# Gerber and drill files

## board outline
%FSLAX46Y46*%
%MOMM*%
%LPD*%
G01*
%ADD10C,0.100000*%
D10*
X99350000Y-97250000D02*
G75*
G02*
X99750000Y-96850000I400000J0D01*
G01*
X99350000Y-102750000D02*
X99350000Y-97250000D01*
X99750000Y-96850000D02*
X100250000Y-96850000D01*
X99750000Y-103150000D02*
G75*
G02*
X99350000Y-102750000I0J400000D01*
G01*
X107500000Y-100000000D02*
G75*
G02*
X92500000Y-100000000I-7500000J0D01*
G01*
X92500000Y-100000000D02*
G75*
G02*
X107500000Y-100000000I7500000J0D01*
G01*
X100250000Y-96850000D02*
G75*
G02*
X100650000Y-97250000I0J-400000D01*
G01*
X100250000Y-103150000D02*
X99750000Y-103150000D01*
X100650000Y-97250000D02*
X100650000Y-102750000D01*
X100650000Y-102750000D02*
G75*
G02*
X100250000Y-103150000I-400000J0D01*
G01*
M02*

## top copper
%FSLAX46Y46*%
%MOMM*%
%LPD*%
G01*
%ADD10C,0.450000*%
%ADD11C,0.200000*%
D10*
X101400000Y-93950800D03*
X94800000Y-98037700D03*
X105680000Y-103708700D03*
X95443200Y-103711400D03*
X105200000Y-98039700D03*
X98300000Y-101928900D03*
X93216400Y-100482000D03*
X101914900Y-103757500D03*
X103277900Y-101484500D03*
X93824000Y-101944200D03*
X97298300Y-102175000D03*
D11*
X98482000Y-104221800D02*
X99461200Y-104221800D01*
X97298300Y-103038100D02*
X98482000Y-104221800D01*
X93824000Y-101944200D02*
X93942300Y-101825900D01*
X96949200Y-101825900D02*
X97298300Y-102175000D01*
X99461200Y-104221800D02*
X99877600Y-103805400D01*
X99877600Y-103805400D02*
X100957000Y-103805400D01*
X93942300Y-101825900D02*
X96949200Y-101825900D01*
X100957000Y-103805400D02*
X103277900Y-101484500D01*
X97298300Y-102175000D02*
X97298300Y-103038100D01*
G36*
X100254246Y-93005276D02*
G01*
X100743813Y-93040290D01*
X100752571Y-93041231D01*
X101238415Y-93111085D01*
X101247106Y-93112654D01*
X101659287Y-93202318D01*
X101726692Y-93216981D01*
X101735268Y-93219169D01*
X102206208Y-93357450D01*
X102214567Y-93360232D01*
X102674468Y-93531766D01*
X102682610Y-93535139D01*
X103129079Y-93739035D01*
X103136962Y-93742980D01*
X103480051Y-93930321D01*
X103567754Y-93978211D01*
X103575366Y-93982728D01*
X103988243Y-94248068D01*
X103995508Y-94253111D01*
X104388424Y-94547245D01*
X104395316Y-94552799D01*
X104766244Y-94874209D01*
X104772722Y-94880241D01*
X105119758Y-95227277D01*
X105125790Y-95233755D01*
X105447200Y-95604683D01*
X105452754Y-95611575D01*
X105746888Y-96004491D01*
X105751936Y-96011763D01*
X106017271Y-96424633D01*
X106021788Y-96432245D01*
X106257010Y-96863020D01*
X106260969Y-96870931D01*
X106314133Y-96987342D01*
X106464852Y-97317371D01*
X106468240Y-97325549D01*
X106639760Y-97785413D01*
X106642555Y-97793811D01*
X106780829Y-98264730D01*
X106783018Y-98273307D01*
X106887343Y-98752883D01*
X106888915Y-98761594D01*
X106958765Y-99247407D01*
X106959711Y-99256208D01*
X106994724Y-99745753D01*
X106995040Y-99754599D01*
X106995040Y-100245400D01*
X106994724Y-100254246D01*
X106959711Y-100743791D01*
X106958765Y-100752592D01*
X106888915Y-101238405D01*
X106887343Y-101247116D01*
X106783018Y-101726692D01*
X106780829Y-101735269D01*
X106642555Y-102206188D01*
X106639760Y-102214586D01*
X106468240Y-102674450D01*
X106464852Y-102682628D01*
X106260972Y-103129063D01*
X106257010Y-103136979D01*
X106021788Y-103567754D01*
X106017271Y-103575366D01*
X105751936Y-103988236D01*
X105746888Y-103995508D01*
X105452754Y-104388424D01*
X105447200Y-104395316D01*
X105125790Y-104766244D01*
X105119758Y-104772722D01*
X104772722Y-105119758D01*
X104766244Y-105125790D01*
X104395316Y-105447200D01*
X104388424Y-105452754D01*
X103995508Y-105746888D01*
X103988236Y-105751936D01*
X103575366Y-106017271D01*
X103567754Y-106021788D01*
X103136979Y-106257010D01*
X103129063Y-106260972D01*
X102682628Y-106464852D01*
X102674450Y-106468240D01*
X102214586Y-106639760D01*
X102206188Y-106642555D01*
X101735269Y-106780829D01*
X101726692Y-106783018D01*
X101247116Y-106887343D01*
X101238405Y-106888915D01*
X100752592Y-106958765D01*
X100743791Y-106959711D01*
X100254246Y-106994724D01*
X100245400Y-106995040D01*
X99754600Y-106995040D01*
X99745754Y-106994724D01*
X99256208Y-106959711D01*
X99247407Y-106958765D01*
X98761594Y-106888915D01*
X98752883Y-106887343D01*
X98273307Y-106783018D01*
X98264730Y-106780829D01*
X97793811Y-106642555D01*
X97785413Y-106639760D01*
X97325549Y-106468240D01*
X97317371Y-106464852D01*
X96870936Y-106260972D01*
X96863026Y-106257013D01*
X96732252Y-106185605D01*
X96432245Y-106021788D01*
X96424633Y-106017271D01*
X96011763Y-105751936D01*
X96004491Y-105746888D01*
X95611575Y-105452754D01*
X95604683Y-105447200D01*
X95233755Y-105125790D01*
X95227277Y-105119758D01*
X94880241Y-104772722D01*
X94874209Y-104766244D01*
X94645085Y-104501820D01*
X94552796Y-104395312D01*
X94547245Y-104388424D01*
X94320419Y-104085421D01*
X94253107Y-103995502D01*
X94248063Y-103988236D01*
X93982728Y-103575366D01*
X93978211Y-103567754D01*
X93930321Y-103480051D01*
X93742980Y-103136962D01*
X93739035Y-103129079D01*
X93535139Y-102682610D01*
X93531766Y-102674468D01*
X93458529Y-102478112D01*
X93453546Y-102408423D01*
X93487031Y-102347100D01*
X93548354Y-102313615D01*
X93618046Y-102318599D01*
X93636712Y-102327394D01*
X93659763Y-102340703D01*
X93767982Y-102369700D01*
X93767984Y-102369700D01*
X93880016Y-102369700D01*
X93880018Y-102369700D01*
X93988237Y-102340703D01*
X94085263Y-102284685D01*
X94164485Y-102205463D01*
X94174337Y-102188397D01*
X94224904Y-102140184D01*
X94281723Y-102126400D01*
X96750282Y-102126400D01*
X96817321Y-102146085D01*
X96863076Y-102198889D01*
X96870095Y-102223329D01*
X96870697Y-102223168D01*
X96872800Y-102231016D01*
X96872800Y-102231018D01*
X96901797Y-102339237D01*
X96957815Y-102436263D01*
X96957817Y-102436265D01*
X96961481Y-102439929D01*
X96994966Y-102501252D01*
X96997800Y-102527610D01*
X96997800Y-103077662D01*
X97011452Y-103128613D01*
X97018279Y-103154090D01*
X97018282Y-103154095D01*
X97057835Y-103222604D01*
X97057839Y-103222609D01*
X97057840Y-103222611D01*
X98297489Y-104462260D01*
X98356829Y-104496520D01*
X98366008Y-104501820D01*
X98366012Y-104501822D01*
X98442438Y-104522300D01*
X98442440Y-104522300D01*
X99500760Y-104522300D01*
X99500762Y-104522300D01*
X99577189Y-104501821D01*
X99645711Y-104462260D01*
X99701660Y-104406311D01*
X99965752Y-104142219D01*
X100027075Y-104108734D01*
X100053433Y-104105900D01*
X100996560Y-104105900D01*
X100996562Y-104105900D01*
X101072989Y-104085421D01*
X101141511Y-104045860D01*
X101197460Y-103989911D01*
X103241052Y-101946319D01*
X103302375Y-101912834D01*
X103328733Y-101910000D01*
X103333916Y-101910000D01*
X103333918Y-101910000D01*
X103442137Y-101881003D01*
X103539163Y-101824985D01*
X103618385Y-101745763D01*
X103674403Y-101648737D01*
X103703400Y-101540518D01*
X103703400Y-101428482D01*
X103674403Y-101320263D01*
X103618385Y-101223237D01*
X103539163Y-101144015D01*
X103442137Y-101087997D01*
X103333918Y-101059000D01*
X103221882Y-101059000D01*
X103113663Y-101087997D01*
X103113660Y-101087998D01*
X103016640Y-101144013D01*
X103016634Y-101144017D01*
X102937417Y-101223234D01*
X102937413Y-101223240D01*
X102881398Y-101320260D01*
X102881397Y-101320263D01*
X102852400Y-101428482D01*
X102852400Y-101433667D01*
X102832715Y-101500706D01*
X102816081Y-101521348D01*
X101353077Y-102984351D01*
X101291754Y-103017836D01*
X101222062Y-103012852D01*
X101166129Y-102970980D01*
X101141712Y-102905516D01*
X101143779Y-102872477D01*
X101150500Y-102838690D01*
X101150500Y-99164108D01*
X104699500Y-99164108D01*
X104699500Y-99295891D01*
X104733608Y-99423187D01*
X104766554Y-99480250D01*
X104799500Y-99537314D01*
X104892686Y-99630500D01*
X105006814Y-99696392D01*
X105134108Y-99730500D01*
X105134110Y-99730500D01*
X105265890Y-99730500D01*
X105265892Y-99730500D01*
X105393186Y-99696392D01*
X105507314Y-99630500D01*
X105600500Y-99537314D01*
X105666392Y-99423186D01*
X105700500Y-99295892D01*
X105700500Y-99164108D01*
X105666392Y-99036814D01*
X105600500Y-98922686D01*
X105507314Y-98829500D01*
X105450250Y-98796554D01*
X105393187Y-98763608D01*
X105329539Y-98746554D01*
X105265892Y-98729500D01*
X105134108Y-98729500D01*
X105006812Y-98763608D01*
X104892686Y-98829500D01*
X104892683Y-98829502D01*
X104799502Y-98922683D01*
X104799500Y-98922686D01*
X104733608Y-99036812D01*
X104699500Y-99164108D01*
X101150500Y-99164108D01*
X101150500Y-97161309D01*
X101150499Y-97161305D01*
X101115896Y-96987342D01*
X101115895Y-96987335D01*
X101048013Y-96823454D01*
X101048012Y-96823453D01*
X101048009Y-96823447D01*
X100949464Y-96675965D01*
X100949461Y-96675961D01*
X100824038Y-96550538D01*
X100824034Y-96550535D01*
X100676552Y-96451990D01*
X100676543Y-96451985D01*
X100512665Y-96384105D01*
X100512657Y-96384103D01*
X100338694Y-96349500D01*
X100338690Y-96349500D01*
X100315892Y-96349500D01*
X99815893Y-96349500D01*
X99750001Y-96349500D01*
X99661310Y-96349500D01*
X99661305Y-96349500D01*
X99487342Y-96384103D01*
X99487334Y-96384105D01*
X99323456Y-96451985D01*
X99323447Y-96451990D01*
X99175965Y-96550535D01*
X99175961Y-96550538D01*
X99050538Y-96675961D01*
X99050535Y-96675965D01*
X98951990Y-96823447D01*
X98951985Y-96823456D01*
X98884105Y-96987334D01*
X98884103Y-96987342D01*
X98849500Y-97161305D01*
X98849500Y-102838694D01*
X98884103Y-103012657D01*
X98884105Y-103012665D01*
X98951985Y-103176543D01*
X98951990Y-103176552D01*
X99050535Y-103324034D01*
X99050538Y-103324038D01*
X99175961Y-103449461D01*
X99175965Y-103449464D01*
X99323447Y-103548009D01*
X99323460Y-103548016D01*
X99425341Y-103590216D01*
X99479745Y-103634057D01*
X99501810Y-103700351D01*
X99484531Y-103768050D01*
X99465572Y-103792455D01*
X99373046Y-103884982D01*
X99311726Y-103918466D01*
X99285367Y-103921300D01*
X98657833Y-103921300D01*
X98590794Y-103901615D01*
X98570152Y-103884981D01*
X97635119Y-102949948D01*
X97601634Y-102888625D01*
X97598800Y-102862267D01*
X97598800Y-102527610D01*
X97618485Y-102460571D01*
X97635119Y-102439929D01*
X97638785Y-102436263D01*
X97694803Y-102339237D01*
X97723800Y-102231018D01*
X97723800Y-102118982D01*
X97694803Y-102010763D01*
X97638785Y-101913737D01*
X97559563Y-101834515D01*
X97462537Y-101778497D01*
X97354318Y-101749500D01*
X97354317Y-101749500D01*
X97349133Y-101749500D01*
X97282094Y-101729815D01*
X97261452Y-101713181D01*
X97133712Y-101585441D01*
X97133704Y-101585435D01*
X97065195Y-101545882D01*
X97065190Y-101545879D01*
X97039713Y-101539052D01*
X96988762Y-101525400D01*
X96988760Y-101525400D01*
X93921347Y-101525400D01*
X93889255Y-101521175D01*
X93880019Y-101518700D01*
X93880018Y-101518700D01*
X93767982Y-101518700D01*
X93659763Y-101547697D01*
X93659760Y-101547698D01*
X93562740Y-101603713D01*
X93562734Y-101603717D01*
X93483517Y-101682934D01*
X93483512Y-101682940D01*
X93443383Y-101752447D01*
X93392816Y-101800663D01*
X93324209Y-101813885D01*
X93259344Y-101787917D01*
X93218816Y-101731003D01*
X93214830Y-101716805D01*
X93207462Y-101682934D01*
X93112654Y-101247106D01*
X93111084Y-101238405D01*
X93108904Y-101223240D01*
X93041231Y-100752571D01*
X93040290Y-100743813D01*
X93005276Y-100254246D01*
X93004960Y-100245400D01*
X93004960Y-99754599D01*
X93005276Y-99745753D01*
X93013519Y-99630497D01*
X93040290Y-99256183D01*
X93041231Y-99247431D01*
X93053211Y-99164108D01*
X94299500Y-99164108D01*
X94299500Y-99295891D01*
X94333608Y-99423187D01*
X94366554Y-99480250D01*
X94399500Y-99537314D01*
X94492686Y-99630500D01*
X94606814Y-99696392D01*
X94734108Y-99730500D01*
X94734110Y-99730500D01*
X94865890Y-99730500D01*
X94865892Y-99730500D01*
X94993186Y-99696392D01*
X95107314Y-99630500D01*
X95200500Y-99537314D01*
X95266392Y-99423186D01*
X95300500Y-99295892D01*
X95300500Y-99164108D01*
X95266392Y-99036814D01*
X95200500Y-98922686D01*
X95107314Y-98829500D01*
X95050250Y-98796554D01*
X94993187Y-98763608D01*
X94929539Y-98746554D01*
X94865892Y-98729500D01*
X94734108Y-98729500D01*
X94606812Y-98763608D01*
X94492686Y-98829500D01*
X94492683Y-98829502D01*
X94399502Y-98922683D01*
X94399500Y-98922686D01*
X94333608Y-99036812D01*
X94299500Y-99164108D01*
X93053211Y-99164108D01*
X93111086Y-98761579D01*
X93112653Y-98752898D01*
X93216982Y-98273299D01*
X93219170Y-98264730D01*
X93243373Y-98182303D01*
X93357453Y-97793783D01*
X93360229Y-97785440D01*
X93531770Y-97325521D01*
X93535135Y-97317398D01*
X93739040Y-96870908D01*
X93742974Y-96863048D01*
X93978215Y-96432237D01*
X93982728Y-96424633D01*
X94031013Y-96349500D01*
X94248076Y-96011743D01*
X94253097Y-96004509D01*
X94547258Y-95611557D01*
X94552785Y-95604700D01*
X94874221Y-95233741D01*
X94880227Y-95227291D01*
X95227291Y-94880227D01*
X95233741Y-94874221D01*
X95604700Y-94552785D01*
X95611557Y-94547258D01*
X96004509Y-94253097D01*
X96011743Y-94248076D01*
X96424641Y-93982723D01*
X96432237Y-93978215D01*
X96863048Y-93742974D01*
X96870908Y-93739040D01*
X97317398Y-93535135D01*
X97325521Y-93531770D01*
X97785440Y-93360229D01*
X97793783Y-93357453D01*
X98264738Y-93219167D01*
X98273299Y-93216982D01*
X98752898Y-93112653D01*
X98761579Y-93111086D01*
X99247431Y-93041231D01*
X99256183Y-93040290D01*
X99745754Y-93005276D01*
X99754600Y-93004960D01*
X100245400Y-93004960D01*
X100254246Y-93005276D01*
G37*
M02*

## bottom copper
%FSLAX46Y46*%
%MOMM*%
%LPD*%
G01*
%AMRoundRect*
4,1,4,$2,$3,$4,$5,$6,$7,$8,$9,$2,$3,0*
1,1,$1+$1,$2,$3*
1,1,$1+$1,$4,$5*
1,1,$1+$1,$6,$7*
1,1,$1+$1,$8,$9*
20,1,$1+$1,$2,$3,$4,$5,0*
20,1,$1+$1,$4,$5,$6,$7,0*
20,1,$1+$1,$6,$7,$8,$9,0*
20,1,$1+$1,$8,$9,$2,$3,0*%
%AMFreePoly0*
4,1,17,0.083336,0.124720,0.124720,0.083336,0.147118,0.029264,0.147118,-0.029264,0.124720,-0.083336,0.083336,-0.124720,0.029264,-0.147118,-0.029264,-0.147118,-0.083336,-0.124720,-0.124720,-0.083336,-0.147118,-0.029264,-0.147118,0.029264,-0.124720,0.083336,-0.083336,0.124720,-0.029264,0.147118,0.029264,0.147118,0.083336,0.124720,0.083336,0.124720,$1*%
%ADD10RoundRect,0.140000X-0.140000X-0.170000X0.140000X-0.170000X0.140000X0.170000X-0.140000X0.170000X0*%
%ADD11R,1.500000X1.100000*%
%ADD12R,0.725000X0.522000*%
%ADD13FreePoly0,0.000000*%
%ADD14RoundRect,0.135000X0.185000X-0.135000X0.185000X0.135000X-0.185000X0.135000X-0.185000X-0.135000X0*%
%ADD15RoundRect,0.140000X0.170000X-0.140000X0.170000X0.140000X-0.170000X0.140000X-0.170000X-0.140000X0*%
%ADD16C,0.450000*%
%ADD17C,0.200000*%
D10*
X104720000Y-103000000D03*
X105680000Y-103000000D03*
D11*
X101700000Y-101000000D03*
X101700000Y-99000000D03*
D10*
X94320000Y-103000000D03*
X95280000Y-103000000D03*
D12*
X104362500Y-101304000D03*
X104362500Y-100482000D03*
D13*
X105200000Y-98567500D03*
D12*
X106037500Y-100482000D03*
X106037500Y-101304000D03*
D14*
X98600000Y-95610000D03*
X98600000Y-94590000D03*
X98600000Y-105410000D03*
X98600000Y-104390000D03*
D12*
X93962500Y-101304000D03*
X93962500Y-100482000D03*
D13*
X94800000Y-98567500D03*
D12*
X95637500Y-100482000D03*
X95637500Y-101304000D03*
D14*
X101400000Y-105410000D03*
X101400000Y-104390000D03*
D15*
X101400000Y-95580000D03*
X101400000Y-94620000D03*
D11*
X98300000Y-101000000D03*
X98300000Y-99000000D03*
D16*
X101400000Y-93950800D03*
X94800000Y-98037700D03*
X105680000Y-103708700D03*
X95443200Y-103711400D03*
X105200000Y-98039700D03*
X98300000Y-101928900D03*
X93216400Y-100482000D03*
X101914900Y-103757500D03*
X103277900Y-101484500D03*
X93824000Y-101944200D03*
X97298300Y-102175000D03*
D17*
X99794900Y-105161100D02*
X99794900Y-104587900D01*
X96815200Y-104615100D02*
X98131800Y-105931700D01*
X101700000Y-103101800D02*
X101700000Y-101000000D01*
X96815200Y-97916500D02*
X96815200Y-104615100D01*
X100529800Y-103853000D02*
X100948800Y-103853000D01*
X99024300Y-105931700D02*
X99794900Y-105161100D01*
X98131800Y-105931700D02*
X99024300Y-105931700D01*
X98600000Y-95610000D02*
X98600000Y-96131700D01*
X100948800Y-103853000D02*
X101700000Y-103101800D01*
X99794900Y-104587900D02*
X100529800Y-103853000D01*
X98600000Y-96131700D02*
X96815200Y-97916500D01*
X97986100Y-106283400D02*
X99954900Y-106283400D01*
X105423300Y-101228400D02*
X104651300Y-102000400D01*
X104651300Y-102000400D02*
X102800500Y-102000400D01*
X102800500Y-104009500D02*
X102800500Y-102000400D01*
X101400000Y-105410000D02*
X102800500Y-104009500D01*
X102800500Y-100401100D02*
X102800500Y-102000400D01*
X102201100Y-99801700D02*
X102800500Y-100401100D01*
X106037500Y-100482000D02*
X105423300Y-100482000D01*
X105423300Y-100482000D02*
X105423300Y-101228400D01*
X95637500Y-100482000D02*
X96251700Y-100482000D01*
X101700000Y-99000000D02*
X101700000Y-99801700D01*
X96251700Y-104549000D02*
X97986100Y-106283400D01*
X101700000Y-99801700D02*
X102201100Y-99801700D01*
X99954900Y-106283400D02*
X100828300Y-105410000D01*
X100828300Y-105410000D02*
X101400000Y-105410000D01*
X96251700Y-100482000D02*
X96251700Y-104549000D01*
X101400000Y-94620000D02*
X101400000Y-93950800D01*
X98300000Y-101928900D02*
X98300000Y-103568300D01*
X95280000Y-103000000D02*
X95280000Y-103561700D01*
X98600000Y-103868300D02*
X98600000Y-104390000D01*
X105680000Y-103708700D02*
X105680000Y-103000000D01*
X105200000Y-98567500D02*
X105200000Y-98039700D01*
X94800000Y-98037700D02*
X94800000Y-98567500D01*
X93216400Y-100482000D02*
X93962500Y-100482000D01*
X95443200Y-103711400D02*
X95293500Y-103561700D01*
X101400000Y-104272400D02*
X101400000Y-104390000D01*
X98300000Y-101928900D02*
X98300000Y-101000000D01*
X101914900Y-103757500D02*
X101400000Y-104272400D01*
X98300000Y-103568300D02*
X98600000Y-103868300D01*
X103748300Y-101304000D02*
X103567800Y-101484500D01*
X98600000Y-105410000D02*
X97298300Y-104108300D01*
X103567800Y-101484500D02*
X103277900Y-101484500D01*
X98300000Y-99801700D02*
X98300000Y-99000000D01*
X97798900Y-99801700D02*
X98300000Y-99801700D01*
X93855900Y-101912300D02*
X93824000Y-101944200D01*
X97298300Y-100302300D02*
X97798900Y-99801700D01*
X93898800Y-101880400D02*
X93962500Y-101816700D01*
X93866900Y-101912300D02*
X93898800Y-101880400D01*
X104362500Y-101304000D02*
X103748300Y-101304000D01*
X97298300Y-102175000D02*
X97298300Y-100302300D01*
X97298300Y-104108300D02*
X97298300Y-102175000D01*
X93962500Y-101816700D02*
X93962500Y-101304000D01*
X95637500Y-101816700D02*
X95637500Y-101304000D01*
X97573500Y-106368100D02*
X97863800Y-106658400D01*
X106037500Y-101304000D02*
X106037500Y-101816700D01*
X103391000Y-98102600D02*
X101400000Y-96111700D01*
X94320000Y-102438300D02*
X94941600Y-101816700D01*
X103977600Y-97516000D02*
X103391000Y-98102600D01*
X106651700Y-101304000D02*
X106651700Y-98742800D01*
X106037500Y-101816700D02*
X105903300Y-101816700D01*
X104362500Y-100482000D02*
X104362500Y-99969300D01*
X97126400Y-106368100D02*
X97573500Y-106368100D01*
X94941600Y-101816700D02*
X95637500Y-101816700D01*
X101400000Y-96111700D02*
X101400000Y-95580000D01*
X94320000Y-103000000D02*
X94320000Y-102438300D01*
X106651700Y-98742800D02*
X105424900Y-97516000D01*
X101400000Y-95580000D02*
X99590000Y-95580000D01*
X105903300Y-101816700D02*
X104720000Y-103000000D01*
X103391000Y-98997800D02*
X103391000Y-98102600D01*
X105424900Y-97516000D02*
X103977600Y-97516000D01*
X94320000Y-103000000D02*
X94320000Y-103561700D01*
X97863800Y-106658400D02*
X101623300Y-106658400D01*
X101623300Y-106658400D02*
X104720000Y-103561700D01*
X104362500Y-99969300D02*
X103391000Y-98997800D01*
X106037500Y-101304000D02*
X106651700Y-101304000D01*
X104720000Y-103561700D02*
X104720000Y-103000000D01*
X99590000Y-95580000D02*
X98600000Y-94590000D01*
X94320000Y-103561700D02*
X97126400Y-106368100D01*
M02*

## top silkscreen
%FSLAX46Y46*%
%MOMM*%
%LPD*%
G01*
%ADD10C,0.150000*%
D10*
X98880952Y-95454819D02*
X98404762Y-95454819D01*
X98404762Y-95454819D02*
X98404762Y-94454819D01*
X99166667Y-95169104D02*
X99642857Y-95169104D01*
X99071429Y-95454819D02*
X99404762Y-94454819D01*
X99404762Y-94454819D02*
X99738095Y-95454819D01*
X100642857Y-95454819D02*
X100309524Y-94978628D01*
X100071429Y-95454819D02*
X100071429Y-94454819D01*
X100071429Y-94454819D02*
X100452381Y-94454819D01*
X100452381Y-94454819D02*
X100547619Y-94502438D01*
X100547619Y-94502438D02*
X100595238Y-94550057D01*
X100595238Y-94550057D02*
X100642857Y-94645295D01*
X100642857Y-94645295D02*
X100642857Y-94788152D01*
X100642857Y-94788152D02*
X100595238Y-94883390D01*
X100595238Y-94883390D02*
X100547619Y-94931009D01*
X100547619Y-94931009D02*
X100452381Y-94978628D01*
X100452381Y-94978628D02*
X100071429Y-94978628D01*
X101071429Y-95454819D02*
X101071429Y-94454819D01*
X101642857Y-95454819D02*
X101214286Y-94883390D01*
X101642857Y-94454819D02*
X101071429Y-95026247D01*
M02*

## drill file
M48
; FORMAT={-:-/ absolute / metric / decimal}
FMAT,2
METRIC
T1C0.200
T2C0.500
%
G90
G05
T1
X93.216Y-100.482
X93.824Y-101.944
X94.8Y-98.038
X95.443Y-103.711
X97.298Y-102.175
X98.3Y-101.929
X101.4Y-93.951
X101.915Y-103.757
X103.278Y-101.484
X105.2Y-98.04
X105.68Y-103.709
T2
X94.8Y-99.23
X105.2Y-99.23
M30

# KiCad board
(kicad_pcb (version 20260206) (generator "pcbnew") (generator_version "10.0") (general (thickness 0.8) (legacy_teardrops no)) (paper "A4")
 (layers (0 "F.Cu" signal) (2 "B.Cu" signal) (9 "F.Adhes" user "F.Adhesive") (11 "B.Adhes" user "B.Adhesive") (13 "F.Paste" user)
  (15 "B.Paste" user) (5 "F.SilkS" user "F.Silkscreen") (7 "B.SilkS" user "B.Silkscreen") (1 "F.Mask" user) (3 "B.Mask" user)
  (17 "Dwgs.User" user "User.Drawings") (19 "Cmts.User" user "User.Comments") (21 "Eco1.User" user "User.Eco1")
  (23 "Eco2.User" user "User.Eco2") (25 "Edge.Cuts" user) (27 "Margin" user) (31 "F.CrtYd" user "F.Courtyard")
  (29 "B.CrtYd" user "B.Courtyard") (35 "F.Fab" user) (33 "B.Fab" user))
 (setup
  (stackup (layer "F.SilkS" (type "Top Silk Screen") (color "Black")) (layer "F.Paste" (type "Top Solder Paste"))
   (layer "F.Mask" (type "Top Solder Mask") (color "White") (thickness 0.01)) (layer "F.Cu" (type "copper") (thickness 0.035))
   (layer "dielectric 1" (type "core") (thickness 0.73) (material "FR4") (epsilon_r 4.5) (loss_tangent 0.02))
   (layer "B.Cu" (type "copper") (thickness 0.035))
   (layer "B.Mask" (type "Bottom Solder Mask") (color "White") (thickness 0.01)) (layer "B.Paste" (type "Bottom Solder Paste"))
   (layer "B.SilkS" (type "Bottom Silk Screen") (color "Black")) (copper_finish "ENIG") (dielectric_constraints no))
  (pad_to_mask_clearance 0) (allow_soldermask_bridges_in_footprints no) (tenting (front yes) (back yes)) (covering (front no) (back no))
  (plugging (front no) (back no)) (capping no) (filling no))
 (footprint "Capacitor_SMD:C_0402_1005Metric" (layer "B.Cu") (at 105.2 103)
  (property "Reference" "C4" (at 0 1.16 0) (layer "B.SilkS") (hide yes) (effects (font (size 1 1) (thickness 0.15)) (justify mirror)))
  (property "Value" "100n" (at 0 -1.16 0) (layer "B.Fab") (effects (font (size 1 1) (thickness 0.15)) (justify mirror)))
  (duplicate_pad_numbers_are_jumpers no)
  (pad "1" smd roundrect (at -0.48 0) (size 0.56 0.62) (layers "B.Cu" "B.Mask" "B.Paste") (roundrect_rratio 0.25) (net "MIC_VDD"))
  (pad "2" smd roundrect (at 0.48 0) (size 0.56 0.62) (layers "B.Cu" "B.Mask" "B.Paste") (roundrect_rratio 0.25) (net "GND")))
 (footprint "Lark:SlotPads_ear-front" (layer "B.Cu") (at 100 100)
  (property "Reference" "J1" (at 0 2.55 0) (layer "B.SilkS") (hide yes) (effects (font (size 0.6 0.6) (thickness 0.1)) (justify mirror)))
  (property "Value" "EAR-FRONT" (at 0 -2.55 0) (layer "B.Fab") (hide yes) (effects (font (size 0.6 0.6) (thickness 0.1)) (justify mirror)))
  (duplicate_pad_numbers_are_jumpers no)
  (pad "1" smd rect (at 1.7 1) (size 1.5 1.1) (layers "B.Cu" "B.Mask") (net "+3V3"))
  (pad "2" smd rect (at 1.7 -1) (size 1.5 1.1) (layers "B.Cu" "B.Mask") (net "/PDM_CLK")))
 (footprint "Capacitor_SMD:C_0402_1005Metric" (layer "B.Cu") (at 94.8 103)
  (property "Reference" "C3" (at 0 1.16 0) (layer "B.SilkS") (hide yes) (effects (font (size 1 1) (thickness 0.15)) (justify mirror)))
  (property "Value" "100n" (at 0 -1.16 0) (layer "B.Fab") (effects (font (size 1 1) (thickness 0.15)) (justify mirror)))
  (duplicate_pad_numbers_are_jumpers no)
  (pad "1" smd roundrect (at -0.48 0) (size 0.56 0.62) (layers "B.Cu" "B.Mask" "B.Paste") (roundrect_rratio 0.25) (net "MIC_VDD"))
  (pad "2" smd roundrect (at 0.48 0) (size 0.56 0.62) (layers "B.Cu" "B.Mask" "B.Paste") (roundrect_rratio 0.25) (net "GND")))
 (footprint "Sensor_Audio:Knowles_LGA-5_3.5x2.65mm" (layer "B.Cu") (at 105.2 100)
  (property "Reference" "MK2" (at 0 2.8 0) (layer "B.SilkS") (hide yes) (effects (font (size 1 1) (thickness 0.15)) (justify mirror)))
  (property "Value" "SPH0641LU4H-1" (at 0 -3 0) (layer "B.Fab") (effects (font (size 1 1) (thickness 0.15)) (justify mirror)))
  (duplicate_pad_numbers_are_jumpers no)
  (pad "" np_thru_hole circle (at 0 -0.77) (size 0.5 0.5) (drill 0.5) (layers "*.Cu" "*.Mask"))
  (pad "1" smd rect (at -0.8375 1.304) (size 0.725 0.522) (layers "B.Cu" "B.Mask" "B.Paste") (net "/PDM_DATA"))
  (pad "2" smd rect (at -0.8375 0.482) (size 0.725 0.522) (layers "B.Cu" "B.Mask" "B.Paste") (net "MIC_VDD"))
  (pad "3" smd custom (at 0 -1.4325) (size 0.3 0.3) (layers "B.Cu" "B.Mask") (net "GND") (zone_connect 0)
   (options (clearance outline) (anchor circle)) (primitives))
  (pad "4" smd rect (at 0.8375 0.482) (size 0.725 0.522) (layers "B.Cu" "B.Mask" "B.Paste") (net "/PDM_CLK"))
  (pad "5" smd rect (at 0.8375 1.304) (size 0.725 0.522) (layers "B.Cu" "B.Mask" "B.Paste") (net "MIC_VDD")))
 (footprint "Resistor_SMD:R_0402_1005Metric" (layer "B.Cu") (at 98.6 95.1 90)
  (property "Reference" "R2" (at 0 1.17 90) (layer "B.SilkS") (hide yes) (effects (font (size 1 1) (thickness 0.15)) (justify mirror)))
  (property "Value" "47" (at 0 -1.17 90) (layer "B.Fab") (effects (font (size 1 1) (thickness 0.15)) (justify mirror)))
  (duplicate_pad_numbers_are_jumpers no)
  (pad "1" smd roundrect (at -0.51 0 90) (size 0.54 0.64) (layers "B.Cu" "B.Mask" "B.Paste") (roundrect_rratio 0.25) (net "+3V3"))
  (pad "2" smd roundrect (at 0.51 0 90) (size 0.54 0.64) (layers "B.Cu" "B.Mask" "B.Paste") (roundrect_rratio 0.25) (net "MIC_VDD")))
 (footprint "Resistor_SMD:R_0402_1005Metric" (layer "B.Cu") (at 98.6 104.9 90)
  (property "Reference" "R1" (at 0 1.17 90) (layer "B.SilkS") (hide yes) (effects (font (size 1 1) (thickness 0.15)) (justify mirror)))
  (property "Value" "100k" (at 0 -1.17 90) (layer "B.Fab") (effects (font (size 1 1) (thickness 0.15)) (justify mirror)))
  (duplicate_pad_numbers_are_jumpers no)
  (pad "1" smd roundrect (at -0.51 0 90) (size 0.54 0.64) (layers "B.Cu" "B.Mask" "B.Paste") (roundrect_rratio 0.25) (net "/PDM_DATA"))
  (pad "2" smd roundrect (at 0.51 0 90) (size 0.54 0.64) (layers "B.Cu" "B.Mask" "B.Paste") (roundrect_rratio 0.25) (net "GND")))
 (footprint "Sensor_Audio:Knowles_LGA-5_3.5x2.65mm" (layer "B.Cu") (at 94.8 100)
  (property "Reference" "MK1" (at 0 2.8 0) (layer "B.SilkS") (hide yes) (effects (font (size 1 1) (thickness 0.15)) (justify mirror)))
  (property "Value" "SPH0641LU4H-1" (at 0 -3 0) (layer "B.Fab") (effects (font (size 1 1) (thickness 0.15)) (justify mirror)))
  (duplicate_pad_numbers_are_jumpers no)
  (pad "" np_thru_hole circle (at 0 -0.77) (size 0.5 0.5) (drill 0.5) (layers "*.Cu" "*.Mask"))
  (pad "1" smd rect (at -0.8375 1.304) (size 0.725 0.522) (layers "B.Cu" "B.Mask" "B.Paste") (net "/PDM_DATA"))
  (pad "2" smd rect (at -0.8375 0.482) (size 0.725 0.522) (layers "B.Cu" "B.Mask" "B.Paste") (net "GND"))
  (pad "3" smd custom (at 0 -1.4325) (size 0.3 0.3) (layers "B.Cu" "B.Mask") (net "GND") (zone_connect 0)
   (options (clearance outline) (anchor circle)) (primitives))
  (pad "4" smd rect (at 0.8375 0.482) (size 0.725 0.522) (layers "B.Cu" "B.Mask" "B.Paste") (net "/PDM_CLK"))
  (pad "5" smd rect (at 0.8375 1.304) (size 0.725 0.522) (layers "B.Cu" "B.Mask" "B.Paste") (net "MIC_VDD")))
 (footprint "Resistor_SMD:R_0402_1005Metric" (layer "B.Cu") (at 101.4 104.9 90)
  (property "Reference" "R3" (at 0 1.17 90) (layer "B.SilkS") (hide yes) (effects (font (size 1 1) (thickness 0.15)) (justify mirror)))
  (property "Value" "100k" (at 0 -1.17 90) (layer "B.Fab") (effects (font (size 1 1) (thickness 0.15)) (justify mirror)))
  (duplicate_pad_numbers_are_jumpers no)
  (pad "1" smd roundrect (at -0.51 0 90) (size 0.54 0.64) (layers "B.Cu" "B.Mask" "B.Paste") (roundrect_rratio 0.25) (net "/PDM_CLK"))
  (pad "2" smd roundrect (at 0.51 0 90) (size 0.54 0.64) (layers "B.Cu" "B.Mask" "B.Paste") (roundrect_rratio 0.25) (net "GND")))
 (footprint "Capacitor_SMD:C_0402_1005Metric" (layer "B.Cu") (at 101.4 95.1 90)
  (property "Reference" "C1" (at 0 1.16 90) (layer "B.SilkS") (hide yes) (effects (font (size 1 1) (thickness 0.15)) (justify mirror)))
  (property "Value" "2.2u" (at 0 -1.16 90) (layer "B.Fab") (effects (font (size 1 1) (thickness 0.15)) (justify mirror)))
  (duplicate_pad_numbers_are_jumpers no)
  (pad "1" smd roundrect (at -0.48 0 90) (size 0.56 0.62) (layers "B.Cu" "B.Mask" "B.Paste") (roundrect_rratio 0.25) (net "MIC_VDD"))
  (pad "2" smd roundrect (at 0.48 0 90) (size 0.56 0.62) (layers "B.Cu" "B.Mask" "B.Paste") (roundrect_rratio 0.25) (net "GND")))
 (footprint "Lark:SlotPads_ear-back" (layer "B.Cu") (at 100 100)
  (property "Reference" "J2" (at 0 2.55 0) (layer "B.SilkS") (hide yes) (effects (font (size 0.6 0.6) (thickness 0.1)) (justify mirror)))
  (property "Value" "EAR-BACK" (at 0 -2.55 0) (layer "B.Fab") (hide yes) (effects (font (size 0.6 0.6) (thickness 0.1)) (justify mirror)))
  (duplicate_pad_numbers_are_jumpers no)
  (pad "1" smd rect (at -1.7 1) (size 1.5 1.1) (layers "B.Cu" "B.Mask") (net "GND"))
  (pad "2" smd rect (at -1.7 -1) (size 1.5 1.1) (layers "B.Cu" "B.Mask") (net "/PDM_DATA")))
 (gr_arc (start 99.35 97.25) (mid 99.467157 96.967157) (end 99.75 96.85) (stroke (width 0.1) (type default)) (layer "Edge.Cuts"))
 (gr_line (start 99.35 102.75) (end 99.35 97.25) (stroke (width 0.1) (type default)) (layer "Edge.Cuts"))
 (gr_line (start 99.75 96.85) (end 100.25 96.85) (stroke (width 0.1) (type default)) (layer "Edge.Cuts"))
 (gr_arc (start 99.75 103.15) (mid 99.467157 103.032843) (end 99.35 102.75) (stroke (width 0.1) (type default)) (layer "Edge.Cuts"))
 (gr_circle (center 100 100) (end 107.5 100) (stroke (width 0.1) (type default)) (fill no) (layer "Edge.Cuts"))
 (gr_arc (start 100.25 96.85) (mid 100.532843 96.967157) (end 100.65 97.25) (stroke (width 0.1) (type default)) (layer "Edge.Cuts"))
 (gr_line (start 100.25 103.15) (end 99.75 103.15) (stroke (width 0.1) (type default)) (layer "Edge.Cuts"))
 (gr_line (start 100.65 97.25) (end 100.65 102.75) (stroke (width 0.1) (type default)) (layer "Edge.Cuts"))
 (gr_arc (start 100.65 102.75) (mid 100.532843 103.032843) (end 100.25 103.15) (stroke (width 0.1) (type default)) (layer "Edge.Cuts"))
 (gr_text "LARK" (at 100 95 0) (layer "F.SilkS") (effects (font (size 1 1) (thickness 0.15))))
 (segment (start 99.7949 105.1611) (end 99.7949 104.5879) (width 0.2) (layer "B.Cu") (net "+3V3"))
 (segment (start 96.8152 104.6151) (end 98.1318 105.9317) (width 0.2) (layer "B.Cu") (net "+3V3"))
 (segment (start 101.7 103.1018) (end 101.7 101) (width 0.2) (layer "B.Cu") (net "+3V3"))
 (segment (start 96.8152 97.9165) (end 96.8152 104.6151) (width 0.2) (layer "B.Cu") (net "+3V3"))
 (segment (start 100.5298 103.853) (end 100.9488 103.853) (width 0.2) (layer "B.Cu") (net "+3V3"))
 (segment (start 99.0243 105.9317) (end 99.7949 105.1611) (width 0.2) (layer "B.Cu") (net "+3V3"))
 (segment (start 98.1318 105.9317) (end 99.0243 105.9317) (width 0.2) (layer "B.Cu") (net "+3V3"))
 (segment (start 98.6 95.61) (end 98.6 96.1317) (width 0.2) (layer "B.Cu") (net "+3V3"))
 (segment (start 100.9488 103.853) (end 101.7 103.1018) (width 0.2) (layer "B.Cu") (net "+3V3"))
 (segment (start 99.7949 104.5879) (end 100.5298 103.853) (width 0.2) (layer "B.Cu") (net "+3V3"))
 (segment (start 98.6 96.1317) (end 96.8152 97.9165) (width 0.2) (layer "B.Cu") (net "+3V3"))
 (segment (start 97.9861 106.2834) (end 99.9549 106.2834) (width 0.2) (layer "B.Cu") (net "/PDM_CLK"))
 (segment (start 105.4233 101.2284) (end 104.6513 102.0004) (width 0.2) (layer "B.Cu") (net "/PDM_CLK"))
 (segment (start 104.6513 102.0004) (end 102.8005 102.0004) (width 0.2) (layer "B.Cu") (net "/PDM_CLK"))
 (segment (start 102.8005 104.0095) (end 102.8005 102.0004) (width 0.2) (layer "B.Cu") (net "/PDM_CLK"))
 (segment (start 101.4 105.41) (end 102.8005 104.0095) (width 0.2) (layer "B.Cu") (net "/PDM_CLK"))
 (segment (start 102.8005 100.4011) (end 102.8005 102.0004) (width 0.2) (layer "B.Cu") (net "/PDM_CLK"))
 (segment (start 102.2011 99.8017) (end 102.8005 100.4011) (width 0.2) (layer "B.Cu") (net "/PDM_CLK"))
 (segment (start 106.0375 100.482) (end 105.4233 100.482) (width 0.2) (layer "B.Cu") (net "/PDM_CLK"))
 (segment (start 105.4233 100.482) (end 105.4233 101.2284) (width 0.2) (layer "B.Cu") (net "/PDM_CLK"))
 (segment (start 95.6375 100.482) (end 96.2517 100.482) (width 0.2) (layer "B.Cu") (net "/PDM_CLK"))
 (segment (start 101.7 99) (end 101.7 99.8017) (width 0.2) (layer "B.Cu") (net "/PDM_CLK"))
 (segment (start 96.2517 104.549) (end 97.9861 106.2834) (width 0.2) (layer "B.Cu") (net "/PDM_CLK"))
 (segment (start 101.7 99.8017) (end 102.2011 99.8017) (width 0.2) (layer "B.Cu") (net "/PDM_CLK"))
 (segment (start 99.9549 106.2834) (end 100.8283 105.41) (width 0.2) (layer "B.Cu") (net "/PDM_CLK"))
 (segment (start 100.8283 105.41) (end 101.4 105.41) (width 0.2) (layer "B.Cu") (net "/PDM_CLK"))
 (segment (start 96.2517 100.482) (end 96.2517 104.549) (width 0.2) (layer "B.Cu") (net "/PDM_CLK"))
 (via (at 101.4 93.9508) (size 0.45) (drill 0.2) (layers "F.Cu" "B.Cu") (capping no) (covering (front no) (back no))
  (plugging (front no) (back no)) (filling no) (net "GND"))
 (via (at 94.8 98.0377) (size 0.45) (drill 0.2) (layers "F.Cu" "B.Cu") (capping no) (covering (front no) (back no))
  (plugging (front no) (back no)) (filling no) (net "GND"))
 (via (at 105.68 103.7087) (size 0.45) (drill 0.2) (layers "F.Cu" "B.Cu") (capping no) (covering (front no) (back no))
  (plugging (front no) (back no)) (filling no) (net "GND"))
 (via (at 95.4432 103.7114) (size 0.45) (drill 0.2) (layers "F.Cu" "B.Cu") (capping no) (covering (front no) (back no))
  (plugging (front no) (back no)) (filling no) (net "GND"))
 (via (at 105.2 98.0397) (size 0.45) (drill 0.2) (layers "F.Cu" "B.Cu") (capping no) (covering (front no) (back no))
  (plugging (front no) (back no)) (filling no) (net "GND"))
 (via (at 98.3 101.9289) (size 0.45) (drill 0.2) (layers "F.Cu" "B.Cu") (capping no) (covering (front no) (back no))
  (plugging (front no) (back no)) (filling no) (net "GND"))
 (via (at 93.2164 100.482) (size 0.45) (drill 0.2) (layers "F.Cu" "B.Cu") (capping no) (covering (front no) (back no))
  (plugging (front no) (back no)) (filling no) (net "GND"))
 (via (at 101.9149 103.7575) (size 0.45) (drill 0.2) (layers "F.Cu" "B.Cu") (capping no) (covering (front no) (back no))
  (plugging (front no) (back no)) (filling no) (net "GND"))
 (segment (start 101.4 94.62) (end 101.4 93.9508) (width 0.2) (layer "B.Cu") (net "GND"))
 (segment (start 98.3 101.9289) (end 98.3 103.5683) (width 0.2) (layer "B.Cu") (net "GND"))
 (segment (start 95.28 103) (end 95.28 103.5617) (width 0.2) (layer "B.Cu") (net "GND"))
 (segment (start 98.6 103.8683) (end 98.6 104.39) (width 0.2) (layer "B.Cu") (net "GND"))
 (segment (start 105.68 103.7087) (end 105.68 103) (width 0.2) (layer "B.Cu") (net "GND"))
 (segment (start 105.2 98.5675) (end 105.2 98.0397) (width 0.2) (layer "B.Cu") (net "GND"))
 (segment (start 94.8 98.0377) (end 94.8 98.5675) (width 0.2) (layer "B.Cu") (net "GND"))
 (segment (start 93.2164 100.482) (end 93.9625 100.482) (width 0.2) (layer "B.Cu") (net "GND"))
 (segment (start 95.4432 103.7114) (end 95.2935 103.5617) (width 0.2) (layer "B.Cu") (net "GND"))
 (segment (start 101.4 104.2724) (end 101.4 104.39) (width 0.2) (layer "B.Cu") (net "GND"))
 (segment (start 98.3 101.9289) (end 98.3 101) (width 0.2) (layer "B.Cu") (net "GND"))
 (segment (start 101.9149 103.7575) (end 101.4 104.2724) (width 0.2) (layer "B.Cu") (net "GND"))
 (segment (start 98.3 103.5683) (end 98.6 103.8683) (width 0.2) (layer "B.Cu") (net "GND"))
 (segment (start 98.482 104.2218) (end 99.4612 104.2218) (width 0.2) (layer "F.Cu") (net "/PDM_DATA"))
 (segment (start 97.2983 103.0381) (end 98.482 104.2218) (width 0.2) (layer "F.Cu") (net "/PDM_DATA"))
 (segment (start 93.824 101.9442) (end 93.9423 101.8259) (width 0.2) (layer "F.Cu") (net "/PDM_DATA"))
 (segment (start 96.9492 101.8259) (end 97.2983 102.175) (width 0.2) (layer "F.Cu") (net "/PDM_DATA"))
 (segment (start 99.4612 104.2218) (end 99.8776 103.8054) (width 0.2) (layer "F.Cu") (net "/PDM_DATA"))
 (segment (start 99.8776 103.8054) (end 100.957 103.8054) (width 0.2) (layer "F.Cu") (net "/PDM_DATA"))
 (segment (start 93.9423 101.8259) (end 96.9492 101.8259) (width 0.2) (layer "F.Cu") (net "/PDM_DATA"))
 (segment (start 100.957 103.8054) (end 103.2779 101.4845) (width 0.2) (layer "F.Cu") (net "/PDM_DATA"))
 (segment (start 97.2983 102.175) (end 97.2983 103.0381) (width 0.2) (layer "F.Cu") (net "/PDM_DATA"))
 (via (at 103.2779 101.4845) (size 0.45) (drill 0.2) (layers "F.Cu" "B.Cu") (capping no) (covering (front no) (back no))
  (plugging (front no) (back no)) (filling no) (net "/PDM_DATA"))
 (via (at 93.824 101.9442) (size 0.45) (drill 0.2) (layers "F.Cu" "B.Cu") (capping no) (covering (front no) (back no))
  (plugging (front no) (back no)) (filling no) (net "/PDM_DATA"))
 (via (at 97.2983 102.175) (size 0.45) (drill 0.2) (layers "F.Cu" "B.Cu") (capping no) (covering (front no) (back no))
  (plugging (front no) (back no)) (filling no) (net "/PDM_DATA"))
 (segment (start 103.7483 101.304) (end 103.5678 101.4845) (width 0.2) (layer "B.Cu") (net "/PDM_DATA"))
 (segment (start 98.6 105.41) (end 97.2983 104.1083) (width 0.2) (layer "B.Cu") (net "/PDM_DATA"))
 (segment (start 103.5678 101.4845) (end 103.2779 101.4845) (width 0.2) (layer "B.Cu") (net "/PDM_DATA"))
 (segment (start 98.3 99.8017) (end 98.3 99) (width 0.2) (layer "B.Cu") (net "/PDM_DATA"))
 (segment (start 97.7989 99.8017) (end 98.3 99.8017) (width 0.2) (layer "B.Cu") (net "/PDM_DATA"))
 (segment (start 93.8559 101.9123) (end 93.824 101.9442) (width 0.2) (layer "B.Cu") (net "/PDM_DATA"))
 (segment (start 97.2983 100.3023) (end 97.7989 99.8017) (width 0.2) (layer "B.Cu") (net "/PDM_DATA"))
 (segment (start 93.8988 101.8804) (end 93.9625 101.8167) (width 0.2) (layer "B.Cu") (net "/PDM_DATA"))
 (segment (start 93.8669 101.9123) (end 93.8988 101.8804) (width 0.2) (layer "B.Cu") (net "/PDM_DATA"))
 (segment (start 104.3625 101.304) (end 103.7483 101.304) (width 0.2) (layer "B.Cu") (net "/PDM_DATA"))
 (segment (start 97.2983 102.175) (end 97.2983 100.3023) (width 0.2) (layer "B.Cu") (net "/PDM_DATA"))
 (segment (start 97.2983 104.1083) (end 97.2983 102.175) (width 0.2) (layer "B.Cu") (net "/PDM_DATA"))
 (segment (start 93.9625 101.8167) (end 93.9625 101.304) (width 0.2) (layer "B.Cu") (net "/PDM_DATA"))
 (segment (start 95.6375 101.8167) (end 95.6375 101.304) (width 0.2) (layer "B.Cu") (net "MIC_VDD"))
 (segment (start 97.5735 106.3681) (end 97.8638 106.6584) (width 0.2) (layer "B.Cu") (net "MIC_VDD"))
 (segment (start 106.0375 101.304) (end 106.0375 101.8167) (width 0.2) (layer "B.Cu") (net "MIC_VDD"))
 (segment (start 103.391 98.1026) (end 101.4 96.1117) (width 0.2) (layer "B.Cu") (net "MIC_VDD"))
 (segment (start 94.32 102.4383) (end 94.9416 101.8167) (width 0.2) (layer "B.Cu") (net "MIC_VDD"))
 (segment (start 103.9776 97.516) (end 103.391 98.1026) (width 0.2) (layer "B.Cu") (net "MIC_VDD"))
 (segment (start 106.6517 101.304) (end 106.6517 98.7428) (width 0.2) (layer "B.Cu") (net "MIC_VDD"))
 (segment (start 106.0375 101.8167) (end 105.9033 101.8167) (width 0.2) (layer "B.Cu") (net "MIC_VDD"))
 (segment (start 104.3625 100.482) (end 104.3625 99.9693) (width 0.2) (layer "B.Cu") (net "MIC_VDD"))
 (segment (start 97.1264 106.3681) (end 97.5735 106.3681) (width 0.2) (layer "B.Cu") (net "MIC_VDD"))
 (segment (start 94.9416 101.8167) (end 95.6375 101.8167) (width 0.2) (layer "B.Cu") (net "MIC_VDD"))
 (segment (start 101.4 96.1117) (end 101.4 95.58) (width 0.2) (layer "B.Cu") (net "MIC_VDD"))
 (segment (start 94.32 103) (end 94.32 102.4383) (width 0.2) (layer "B.Cu") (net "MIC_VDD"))
 (segment (start 106.6517 98.7428) (end 105.4249 97.516) (width 0.2) (layer "B.Cu") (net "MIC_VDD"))
 (segment (start 101.4 95.58) (end 99.59 95.58) (width 0.2) (layer "B.Cu") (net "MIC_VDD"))
 (segment (start 105.9033 101.8167) (end 104.72 103) (width 0.2) (layer "B.Cu") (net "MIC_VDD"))
 (segment (start 103.391 98.9978) (end 103.391 98.1026) (width 0.2) (layer "B.Cu") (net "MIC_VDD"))
 (segment (start 105.4249 97.516) (end 103.9776 97.516) (width 0.2) (layer "B.Cu") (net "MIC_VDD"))
 (segment (start 94.32 103) (end 94.32 103.5617) (width 0.2) (layer "B.Cu") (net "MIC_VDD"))
 (segment (start 97.8638 106.6584) (end 101.6233 106.6584) (width 0.2) (layer "B.Cu") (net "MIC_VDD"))
 (segment (start 101.6233 106.6584) (end 104.72 103.5617) (width 0.2) (layer "B.Cu") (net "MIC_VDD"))
 (segment (start 104.3625 99.9693) (end 103.391 98.9978) (width 0.2) (layer "B.Cu") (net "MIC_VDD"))
 (segment (start 106.0375 101.304) (end 106.6517 101.304) (width 0.2) (layer "B.Cu") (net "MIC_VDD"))
 (segment (start 104.72 103.5617) (end 104.72 103) (width 0.2) (layer "B.Cu") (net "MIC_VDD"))
 (segment (start 99.59 95.58) (end 98.6 94.59) (width 0.2) (layer "B.Cu") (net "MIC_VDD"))
 (segment (start 94.32 103.5617) (end 97.1264 106.3681) (width 0.2) (layer "B.Cu") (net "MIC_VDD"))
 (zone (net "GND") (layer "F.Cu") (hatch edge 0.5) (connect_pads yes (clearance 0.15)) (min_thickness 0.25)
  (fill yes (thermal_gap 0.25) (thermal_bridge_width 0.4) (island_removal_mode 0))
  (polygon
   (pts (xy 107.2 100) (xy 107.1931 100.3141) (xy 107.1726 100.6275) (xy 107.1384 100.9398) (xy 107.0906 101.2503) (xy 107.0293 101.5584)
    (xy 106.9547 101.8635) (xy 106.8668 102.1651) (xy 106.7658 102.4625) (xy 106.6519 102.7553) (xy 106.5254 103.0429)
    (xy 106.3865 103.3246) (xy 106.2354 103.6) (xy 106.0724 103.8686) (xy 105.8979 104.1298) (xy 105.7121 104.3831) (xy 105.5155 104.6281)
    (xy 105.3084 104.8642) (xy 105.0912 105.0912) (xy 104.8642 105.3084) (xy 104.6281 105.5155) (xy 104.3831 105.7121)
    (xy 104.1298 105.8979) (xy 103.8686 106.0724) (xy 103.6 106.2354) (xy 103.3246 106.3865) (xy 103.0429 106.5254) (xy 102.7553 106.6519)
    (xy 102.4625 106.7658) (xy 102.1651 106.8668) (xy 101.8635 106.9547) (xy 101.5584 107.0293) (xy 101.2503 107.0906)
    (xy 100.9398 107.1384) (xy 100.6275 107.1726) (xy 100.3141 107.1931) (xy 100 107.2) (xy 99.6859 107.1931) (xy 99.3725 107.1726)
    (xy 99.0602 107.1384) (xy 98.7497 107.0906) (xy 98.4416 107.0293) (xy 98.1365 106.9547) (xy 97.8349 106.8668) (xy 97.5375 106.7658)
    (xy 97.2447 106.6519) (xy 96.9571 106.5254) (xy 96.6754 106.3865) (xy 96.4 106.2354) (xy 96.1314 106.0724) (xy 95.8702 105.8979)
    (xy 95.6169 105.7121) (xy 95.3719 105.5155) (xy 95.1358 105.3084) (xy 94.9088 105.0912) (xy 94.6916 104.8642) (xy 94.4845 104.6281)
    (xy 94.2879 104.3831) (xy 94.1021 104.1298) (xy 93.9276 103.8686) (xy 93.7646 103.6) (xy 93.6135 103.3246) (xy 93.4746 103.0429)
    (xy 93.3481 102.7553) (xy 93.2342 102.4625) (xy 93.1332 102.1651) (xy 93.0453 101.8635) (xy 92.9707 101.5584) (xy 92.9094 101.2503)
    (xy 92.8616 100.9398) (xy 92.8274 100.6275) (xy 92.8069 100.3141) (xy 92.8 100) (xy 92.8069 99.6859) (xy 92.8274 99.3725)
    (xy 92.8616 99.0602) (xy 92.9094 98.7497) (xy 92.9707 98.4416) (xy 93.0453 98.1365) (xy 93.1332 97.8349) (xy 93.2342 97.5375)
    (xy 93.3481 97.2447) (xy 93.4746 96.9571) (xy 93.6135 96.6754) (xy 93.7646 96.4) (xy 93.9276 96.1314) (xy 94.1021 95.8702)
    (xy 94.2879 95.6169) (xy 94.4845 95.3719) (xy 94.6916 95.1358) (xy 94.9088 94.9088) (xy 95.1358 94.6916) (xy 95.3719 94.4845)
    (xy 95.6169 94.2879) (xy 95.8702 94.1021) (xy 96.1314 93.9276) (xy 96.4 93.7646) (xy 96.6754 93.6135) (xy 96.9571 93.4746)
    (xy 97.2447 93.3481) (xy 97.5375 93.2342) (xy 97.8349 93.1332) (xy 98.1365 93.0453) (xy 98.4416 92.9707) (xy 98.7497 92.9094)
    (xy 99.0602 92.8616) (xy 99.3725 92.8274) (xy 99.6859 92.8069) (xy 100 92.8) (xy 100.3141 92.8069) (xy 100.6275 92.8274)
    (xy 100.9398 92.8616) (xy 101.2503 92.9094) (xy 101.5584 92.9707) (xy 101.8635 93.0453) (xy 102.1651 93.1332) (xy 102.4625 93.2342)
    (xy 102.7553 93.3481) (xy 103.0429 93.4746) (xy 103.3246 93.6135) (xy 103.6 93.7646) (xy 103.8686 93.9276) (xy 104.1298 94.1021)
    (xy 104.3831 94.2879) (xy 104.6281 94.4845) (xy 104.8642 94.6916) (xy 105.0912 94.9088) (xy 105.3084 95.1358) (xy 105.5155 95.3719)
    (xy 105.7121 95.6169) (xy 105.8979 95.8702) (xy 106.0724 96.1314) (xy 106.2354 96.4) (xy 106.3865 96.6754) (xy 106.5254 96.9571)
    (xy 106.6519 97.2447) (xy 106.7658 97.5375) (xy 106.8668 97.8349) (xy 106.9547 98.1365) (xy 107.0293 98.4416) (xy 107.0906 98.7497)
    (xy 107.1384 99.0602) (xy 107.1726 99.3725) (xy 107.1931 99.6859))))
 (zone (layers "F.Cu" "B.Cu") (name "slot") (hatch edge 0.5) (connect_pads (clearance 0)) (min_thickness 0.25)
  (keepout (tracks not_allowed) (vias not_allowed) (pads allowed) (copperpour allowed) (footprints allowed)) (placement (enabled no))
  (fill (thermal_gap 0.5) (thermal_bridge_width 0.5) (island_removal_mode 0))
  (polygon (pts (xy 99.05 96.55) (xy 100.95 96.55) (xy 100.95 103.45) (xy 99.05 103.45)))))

